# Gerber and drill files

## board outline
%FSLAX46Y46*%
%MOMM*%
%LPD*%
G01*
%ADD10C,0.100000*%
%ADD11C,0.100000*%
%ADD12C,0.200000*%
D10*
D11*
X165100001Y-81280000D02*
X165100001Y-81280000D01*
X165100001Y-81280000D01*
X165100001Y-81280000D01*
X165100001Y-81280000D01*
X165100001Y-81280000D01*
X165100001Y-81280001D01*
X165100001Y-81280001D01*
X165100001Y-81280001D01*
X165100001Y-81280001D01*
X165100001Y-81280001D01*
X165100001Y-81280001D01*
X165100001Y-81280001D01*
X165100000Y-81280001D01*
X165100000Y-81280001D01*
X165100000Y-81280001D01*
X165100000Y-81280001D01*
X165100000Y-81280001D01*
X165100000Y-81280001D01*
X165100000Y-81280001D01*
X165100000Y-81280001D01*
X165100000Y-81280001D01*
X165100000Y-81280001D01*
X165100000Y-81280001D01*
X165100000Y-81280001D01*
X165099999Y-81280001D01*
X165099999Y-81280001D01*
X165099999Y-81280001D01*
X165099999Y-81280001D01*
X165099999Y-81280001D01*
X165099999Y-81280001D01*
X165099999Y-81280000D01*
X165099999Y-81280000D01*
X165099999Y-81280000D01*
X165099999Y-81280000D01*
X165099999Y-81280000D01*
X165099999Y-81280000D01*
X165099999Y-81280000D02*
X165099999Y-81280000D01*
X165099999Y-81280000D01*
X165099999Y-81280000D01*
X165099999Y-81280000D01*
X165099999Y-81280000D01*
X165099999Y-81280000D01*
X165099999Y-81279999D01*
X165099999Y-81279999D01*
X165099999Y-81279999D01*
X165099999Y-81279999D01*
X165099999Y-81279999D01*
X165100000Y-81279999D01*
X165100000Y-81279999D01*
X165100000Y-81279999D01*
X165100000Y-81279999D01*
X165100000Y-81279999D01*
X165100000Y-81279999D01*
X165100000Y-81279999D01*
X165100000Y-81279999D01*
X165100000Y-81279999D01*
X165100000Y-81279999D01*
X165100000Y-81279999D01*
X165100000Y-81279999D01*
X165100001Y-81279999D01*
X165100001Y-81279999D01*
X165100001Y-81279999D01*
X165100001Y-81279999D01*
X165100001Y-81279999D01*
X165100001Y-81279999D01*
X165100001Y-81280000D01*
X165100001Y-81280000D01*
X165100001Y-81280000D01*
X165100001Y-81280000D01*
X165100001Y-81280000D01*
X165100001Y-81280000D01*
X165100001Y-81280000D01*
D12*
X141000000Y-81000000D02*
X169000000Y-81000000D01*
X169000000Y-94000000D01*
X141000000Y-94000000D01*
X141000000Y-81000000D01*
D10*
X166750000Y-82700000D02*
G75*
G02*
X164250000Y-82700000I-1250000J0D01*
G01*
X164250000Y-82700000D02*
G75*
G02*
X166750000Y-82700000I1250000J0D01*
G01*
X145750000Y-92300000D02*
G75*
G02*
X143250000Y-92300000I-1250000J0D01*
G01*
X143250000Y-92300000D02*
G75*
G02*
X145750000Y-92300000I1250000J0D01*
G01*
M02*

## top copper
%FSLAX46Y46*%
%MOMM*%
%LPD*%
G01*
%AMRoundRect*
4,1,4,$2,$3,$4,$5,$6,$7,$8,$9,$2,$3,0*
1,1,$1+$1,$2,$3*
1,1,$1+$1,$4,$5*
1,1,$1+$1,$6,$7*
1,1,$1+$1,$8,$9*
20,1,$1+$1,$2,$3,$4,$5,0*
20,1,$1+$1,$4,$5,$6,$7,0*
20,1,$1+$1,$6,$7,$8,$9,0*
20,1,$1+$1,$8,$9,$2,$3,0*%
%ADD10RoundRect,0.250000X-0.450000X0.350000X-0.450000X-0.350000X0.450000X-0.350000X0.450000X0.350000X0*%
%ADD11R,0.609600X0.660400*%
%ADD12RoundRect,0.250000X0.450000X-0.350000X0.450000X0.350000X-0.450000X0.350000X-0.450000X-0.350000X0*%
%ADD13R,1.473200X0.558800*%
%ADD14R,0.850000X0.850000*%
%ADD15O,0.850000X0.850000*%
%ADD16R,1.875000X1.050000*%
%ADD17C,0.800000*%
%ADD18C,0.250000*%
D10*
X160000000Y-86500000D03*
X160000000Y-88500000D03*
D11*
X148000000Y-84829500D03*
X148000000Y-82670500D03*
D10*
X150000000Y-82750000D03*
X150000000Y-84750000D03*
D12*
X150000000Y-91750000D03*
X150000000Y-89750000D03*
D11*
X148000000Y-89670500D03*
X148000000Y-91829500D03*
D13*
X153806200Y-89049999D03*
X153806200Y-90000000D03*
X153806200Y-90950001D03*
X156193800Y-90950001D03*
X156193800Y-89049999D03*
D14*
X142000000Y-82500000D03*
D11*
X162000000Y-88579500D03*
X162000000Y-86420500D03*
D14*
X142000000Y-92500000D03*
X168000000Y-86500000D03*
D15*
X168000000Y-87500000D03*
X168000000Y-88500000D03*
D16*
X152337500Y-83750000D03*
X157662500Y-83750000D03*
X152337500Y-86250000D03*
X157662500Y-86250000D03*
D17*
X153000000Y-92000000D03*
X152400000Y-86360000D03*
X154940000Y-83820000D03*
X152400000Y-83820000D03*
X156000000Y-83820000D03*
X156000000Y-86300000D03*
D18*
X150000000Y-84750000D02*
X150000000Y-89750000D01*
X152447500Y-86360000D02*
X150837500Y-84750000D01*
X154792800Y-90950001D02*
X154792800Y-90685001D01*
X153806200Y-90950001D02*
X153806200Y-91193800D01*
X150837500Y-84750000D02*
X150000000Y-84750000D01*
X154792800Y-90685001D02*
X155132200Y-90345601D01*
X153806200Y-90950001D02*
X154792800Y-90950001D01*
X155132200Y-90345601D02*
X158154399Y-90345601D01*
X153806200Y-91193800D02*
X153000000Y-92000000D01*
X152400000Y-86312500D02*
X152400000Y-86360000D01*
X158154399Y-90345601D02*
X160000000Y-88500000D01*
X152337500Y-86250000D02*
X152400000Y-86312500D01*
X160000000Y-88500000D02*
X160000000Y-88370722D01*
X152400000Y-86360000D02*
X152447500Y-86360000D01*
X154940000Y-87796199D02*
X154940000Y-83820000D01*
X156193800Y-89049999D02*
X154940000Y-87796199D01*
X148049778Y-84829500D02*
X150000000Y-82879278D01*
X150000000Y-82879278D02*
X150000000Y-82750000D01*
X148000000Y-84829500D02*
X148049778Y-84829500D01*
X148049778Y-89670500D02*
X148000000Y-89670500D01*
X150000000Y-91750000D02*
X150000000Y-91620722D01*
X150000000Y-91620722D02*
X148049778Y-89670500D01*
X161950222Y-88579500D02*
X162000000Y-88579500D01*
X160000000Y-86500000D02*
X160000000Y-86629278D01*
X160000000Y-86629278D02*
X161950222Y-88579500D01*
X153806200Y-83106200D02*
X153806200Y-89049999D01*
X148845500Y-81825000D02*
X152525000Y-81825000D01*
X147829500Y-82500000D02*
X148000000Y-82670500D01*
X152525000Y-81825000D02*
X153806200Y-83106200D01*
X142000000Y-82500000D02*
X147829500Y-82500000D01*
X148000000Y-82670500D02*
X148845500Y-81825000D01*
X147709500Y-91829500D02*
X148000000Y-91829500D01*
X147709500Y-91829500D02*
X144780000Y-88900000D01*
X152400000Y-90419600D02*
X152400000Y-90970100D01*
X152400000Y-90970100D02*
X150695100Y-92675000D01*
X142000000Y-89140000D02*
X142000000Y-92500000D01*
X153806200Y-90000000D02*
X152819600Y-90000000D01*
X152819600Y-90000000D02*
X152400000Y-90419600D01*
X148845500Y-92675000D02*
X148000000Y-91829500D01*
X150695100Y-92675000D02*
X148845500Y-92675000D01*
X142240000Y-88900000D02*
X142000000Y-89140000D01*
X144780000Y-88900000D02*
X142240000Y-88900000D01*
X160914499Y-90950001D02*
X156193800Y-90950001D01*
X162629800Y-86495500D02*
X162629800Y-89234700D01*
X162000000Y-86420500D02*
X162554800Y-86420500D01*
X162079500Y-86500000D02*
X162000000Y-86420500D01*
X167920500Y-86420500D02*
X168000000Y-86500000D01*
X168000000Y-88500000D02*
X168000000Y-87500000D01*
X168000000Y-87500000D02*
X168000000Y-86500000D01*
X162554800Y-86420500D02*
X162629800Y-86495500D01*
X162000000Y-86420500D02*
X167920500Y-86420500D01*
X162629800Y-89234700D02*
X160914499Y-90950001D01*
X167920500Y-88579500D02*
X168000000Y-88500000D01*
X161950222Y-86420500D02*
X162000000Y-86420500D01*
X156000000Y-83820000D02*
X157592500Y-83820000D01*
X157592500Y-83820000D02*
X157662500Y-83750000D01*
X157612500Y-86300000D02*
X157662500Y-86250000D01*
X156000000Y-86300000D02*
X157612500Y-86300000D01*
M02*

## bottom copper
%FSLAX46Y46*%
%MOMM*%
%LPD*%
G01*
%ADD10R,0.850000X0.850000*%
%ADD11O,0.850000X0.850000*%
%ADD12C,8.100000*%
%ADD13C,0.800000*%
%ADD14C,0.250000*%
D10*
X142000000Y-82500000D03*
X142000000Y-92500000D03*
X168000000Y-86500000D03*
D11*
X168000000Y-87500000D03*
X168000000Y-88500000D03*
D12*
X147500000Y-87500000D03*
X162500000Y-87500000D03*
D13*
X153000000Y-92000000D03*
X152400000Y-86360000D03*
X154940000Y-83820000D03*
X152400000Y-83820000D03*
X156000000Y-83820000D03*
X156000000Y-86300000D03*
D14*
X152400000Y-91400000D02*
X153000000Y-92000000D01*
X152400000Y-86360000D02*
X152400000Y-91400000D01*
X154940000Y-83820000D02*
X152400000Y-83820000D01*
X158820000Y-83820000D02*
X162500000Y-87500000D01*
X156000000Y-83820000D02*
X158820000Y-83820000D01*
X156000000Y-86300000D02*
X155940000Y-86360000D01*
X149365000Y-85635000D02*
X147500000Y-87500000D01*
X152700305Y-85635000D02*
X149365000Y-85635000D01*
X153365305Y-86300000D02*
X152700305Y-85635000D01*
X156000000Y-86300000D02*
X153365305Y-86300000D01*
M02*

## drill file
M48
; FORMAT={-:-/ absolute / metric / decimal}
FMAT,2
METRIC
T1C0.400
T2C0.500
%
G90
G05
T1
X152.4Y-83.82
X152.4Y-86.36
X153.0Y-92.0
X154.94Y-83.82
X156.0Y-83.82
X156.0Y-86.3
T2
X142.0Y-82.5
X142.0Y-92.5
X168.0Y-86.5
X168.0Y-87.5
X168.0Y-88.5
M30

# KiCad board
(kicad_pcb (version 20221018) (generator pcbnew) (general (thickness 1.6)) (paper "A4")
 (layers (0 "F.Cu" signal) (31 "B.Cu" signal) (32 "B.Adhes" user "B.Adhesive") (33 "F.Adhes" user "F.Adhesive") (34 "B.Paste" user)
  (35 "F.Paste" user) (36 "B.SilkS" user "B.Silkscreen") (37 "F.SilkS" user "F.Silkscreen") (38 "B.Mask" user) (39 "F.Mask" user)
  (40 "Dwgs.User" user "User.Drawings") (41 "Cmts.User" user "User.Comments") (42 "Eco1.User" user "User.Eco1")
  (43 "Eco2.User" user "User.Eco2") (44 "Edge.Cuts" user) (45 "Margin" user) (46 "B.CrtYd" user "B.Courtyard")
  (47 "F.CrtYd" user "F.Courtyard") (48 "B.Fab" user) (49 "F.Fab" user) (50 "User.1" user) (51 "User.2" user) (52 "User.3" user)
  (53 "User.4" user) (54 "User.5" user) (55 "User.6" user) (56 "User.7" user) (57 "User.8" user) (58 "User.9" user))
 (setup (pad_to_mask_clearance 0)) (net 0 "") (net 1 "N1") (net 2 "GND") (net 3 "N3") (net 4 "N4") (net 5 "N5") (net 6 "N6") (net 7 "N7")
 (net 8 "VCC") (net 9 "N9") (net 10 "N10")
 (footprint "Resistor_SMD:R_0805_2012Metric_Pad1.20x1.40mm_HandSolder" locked (layer "F.Cu") (at 160 87.5 -90)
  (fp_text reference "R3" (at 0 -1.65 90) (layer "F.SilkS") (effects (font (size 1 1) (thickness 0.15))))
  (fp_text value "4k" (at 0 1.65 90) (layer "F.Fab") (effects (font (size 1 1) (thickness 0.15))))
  (pad "1" smd roundrect locked (at -1 0 270) (size 1.2 1.4) (layers "F.Cu" "F.Paste" "F.Mask") (roundrect_rratio 0.208333) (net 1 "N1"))
  (pad "2" smd roundrect locked (at 1 0 270) (size 1.2 1.4) (layers "F.Cu" "F.Paste" "F.Mask") (roundrect_rratio 0.208333) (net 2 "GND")))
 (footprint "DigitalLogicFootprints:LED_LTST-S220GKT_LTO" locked (layer "F.Cu") (at 148 83.75 90)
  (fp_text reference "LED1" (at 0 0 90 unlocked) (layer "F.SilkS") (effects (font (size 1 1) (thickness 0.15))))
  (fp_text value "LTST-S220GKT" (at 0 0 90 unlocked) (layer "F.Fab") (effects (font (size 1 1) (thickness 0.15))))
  (pad "1" smd rect locked (at -1.0795 0 90) (size 0.6604 0.6096) (layers "F.Cu" "F.Paste" "F.Mask") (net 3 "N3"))
  (pad "2" smd rect locked (at 1.0795 0 90) (size 0.6604 0.6096) (layers "F.Cu" "F.Paste" "F.Mask") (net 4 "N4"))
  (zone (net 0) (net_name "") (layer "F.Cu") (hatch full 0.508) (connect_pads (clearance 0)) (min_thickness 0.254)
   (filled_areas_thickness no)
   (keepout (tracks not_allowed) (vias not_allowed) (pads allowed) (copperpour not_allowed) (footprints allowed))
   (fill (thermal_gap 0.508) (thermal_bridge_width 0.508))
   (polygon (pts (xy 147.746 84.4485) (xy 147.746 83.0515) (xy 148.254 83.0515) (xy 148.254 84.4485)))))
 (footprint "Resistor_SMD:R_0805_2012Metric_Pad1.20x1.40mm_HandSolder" (layer "F.Cu") (at 150 83.75 -90)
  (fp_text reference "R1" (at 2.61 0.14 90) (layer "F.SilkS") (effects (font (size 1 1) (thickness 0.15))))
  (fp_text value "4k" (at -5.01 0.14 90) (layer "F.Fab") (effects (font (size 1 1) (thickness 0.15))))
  (pad "1" smd roundrect (at -1 0 270) (size 1.2 1.4) (layers "F.Cu" "F.Paste" "F.Mask") (roundrect_rratio 0.208333) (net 3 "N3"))
  (pad "2" smd roundrect (at 1 0 270) (size 1.2 1.4) (layers "F.Cu" "F.Paste" "F.Mask") (roundrect_rratio 0.208333) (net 2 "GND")))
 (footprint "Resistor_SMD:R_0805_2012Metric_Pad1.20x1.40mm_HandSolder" (layer "F.Cu") (at 150 90.75 90)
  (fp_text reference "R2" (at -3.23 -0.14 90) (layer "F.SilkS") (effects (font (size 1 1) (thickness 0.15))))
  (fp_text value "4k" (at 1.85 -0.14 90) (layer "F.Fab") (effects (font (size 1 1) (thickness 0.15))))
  (pad "1" smd roundrect (at -1 0 90) (size 1.2 1.4) (layers "F.Cu" "F.Paste" "F.Mask") (roundrect_rratio 0.208333) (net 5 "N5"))
  (pad "2" smd roundrect (at 1 0 90) (size 1.2 1.4) (layers "F.Cu" "F.Paste" "F.Mask") (roundrect_rratio 0.208333) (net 2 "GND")))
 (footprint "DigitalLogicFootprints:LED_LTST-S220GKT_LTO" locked (layer "F.Cu") (at 148 90.75 -90)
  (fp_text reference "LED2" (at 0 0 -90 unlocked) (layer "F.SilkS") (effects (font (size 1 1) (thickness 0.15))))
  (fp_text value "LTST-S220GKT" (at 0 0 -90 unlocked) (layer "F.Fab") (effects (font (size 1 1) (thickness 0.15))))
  (pad "1" smd rect locked (at -1.0795 0 270) (size 0.6604 0.6096) (layers "F.Cu" "F.Paste" "F.Mask") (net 5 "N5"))
  (pad "2" smd rect locked (at 1.0795 0 270) (size 0.6604 0.6096) (layers "F.Cu" "F.Paste" "F.Mask") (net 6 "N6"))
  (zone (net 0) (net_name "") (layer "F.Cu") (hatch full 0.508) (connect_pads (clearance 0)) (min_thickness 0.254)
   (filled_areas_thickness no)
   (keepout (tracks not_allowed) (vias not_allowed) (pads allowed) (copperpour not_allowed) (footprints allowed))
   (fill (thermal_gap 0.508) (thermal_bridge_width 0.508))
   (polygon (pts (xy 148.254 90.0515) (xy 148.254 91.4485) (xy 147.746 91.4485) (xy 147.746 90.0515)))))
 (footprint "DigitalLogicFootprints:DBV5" (layer "F.Cu") (at 155 90)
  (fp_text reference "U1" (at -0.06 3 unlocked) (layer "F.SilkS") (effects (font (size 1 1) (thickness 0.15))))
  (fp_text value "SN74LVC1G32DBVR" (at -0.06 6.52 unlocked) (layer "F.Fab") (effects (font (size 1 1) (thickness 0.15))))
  (pad "1" smd rect (at -1.1938 -0.950001) (size 1.4732 0.5588) (layers "F.Cu" "F.Paste" "F.Mask") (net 4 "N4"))
  (pad "2" smd rect (at -1.1938 0) (size 1.4732 0.5588) (layers "F.Cu" "F.Paste" "F.Mask") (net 6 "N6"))
  (pad "3" smd rect (at -1.1938 0.950001) (size 1.4732 0.5588) (layers "F.Cu" "F.Paste" "F.Mask") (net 2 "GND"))
  (pad "4" smd rect (at 1.1938 0.950001) (size 1.4732 0.5588) (layers "F.Cu" "F.Paste" "F.Mask") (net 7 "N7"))
  (pad "5" smd rect (at 1.1938 -0.950001) (size 1.4732 0.5588) (layers "F.Cu" "F.Paste" "F.Mask") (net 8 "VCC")))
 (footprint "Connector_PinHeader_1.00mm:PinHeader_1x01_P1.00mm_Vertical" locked (layer "F.Cu") (at 142 82.5)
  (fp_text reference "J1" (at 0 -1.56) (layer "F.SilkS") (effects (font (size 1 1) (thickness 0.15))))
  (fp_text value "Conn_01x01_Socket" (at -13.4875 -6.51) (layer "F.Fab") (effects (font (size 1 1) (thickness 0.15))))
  (pad "1" thru_hole rect locked (at 0 0) (size 0.85 0.85) (drill 0.5) (layers "*.Cu" "*.Mask") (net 4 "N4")))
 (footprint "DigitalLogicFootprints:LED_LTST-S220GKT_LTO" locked (layer "F.Cu") (at 162 87.5 90)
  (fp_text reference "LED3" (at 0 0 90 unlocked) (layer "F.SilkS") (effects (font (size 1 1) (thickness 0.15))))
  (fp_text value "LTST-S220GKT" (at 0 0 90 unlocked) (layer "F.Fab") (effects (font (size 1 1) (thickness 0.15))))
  (pad "1" smd rect locked (at -1.0795 0 90) (size 0.6604 0.6096) (layers "F.Cu" "F.Paste" "F.Mask") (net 1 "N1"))
  (pad "2" smd rect locked (at 1.0795 0 90) (size 0.6604 0.6096) (layers "F.Cu" "F.Paste" "F.Mask") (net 7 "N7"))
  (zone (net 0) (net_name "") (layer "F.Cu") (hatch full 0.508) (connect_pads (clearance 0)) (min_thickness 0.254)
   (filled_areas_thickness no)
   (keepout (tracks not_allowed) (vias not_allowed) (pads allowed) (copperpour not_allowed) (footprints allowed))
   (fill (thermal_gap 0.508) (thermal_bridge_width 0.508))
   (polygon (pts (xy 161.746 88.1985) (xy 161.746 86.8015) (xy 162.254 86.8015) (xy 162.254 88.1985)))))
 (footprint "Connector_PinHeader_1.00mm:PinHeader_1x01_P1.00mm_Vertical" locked (layer "F.Cu") (at 142 92.5)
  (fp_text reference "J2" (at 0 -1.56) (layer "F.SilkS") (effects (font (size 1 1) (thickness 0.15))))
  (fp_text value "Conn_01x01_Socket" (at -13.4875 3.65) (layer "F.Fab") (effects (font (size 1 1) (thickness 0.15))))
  (pad "1" thru_hole rect locked (at 0 0) (size 0.85 0.85) (drill 0.5) (layers "*.Cu" "*.Mask") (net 6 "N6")))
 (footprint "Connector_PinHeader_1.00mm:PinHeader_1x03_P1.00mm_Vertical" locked (layer "F.Cu") (at 168 86.5)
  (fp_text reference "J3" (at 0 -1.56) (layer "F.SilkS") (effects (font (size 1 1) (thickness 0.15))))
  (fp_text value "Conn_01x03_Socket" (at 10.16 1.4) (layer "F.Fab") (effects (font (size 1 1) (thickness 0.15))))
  (pad "1" thru_hole rect locked (at 0 0) (size 0.85 0.85) (drill 0.5) (layers "*.Cu" "*.Mask") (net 7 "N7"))
  (pad "2" thru_hole oval locked (at 0 1) (size 0.85 0.85) (drill 0.5) (layers "*.Cu" "*.Mask") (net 7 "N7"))
  (pad "3" thru_hole oval locked (at 0 2) (size 0.85 0.85) (drill 0.5) (layers "*.Cu" "*.Mask") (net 7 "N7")))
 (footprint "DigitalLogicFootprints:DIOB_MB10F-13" (layer "F.Cu") (at 155 85)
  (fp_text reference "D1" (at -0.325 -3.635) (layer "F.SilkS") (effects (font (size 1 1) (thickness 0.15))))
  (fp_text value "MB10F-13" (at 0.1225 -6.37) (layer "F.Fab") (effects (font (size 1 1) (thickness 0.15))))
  (pad "1" smd rect (at -2.6625 -1.25) (size 1.875 1.05) (layers "F.Cu" "F.Paste" "F.Mask") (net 8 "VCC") (solder_mask_margin 0.102))
  (pad "2" smd rect (at 2.6625 -1.25 180) (size 1.875 1.05) (layers "F.Cu" "F.Paste" "F.Mask") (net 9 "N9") (solder_mask_margin 0.102))
  (pad "3" smd rect (at -2.6625 1.25) (size 1.875 1.05) (layers "F.Cu" "F.Paste" "F.Mask") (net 2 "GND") (solder_mask_margin 0.102))
  (pad "4" smd rect (at 2.6625 1.25 180) (size 1.875 1.05) (layers "F.Cu" "F.Paste" "F.Mask") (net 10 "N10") (solder_mask_margin 0.102)))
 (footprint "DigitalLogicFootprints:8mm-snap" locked (layer "B.Cu") (at 147.5 87.5 180)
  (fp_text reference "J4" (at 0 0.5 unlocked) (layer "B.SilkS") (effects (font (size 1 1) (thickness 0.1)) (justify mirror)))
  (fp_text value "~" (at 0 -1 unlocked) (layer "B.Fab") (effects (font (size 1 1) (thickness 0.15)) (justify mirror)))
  (pad "1" smd circle locked (at 0 0 180) (size 8.1 8.1) (layers "B.Cu" "B.Paste" "B.Mask") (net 10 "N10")))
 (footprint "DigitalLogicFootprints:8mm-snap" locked (layer "B.Cu") (at 162.5 87.5 180)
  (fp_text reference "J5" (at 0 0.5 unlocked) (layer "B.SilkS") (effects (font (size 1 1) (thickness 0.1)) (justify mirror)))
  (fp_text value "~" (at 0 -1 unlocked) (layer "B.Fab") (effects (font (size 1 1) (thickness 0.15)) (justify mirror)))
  (pad "1" smd circle locked (at 0 0 180) (size 8.1 8.1) (layers "B.Cu" "B.Paste" "B.Mask") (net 9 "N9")))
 (gr_circle (center 165.1 81.28) (end 165.1 81.28) (stroke (width 0.1) (type default)) (fill none) (layer "Edge.Cuts"))
 (gr_rect locked (start 141 81) (end 169 94) (stroke (width 0.2) (type default)) (fill none) (layer "Edge.Cuts"))
 (gr_circle (center 165.5 82.7) (end 166.75 82.7) (stroke (width 0.1) (type default)) (fill none) (layer "Edge.Cuts"))
 (gr_circle (center 144.5 92.3) (end 145.75 92.3) (stroke (width 0.1) (type default)) (fill none) (layer "Edge.Cuts"))
 (segment (start 150 84.75) (end 150 89.75) (width 0.25) (layer "F.Cu") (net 2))
 (segment (start 152.4475 86.36) (end 150.8375 84.75) (width 0.25) (layer "F.Cu") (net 2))
 (segment (start 154.7928 90.950001) (end 154.7928 90.685001) (width 0.25) (layer "F.Cu") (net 2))
 (segment (start 153.8062 90.950001) (end 153.8062 91.1938) (width 0.25) (layer "F.Cu") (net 2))
 (segment (start 150.8375 84.75) (end 150 84.75) (width 0.25) (layer "F.Cu") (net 2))
 (segment (start 154.7928 90.685001) (end 155.1322 90.345601) (width 0.25) (layer "F.Cu") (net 2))
 (segment (start 153.8062 90.950001) (end 154.7928 90.950001) (width 0.25) (layer "F.Cu") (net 2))
 (segment (start 155.1322 90.345601) (end 158.154399 90.345601) (width 0.25) (layer "F.Cu") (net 2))
 (segment (start 153.8062 91.1938) (end 153 92) (width 0.25) (layer "F.Cu") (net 2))
 (segment (start 152.4 86.3125) (end 152.4 86.36) (width 0.25) (layer "F.Cu") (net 2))
 (segment (start 158.154399 90.345601) (end 160 88.5) (width 0.25) (layer "F.Cu") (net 2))
 (segment (start 152.3375 86.25) (end 152.4 86.3125) (width 0.25) (layer "F.Cu") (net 2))
 (segment (start 160 88.5) (end 160 88.370722) (width 0.25) (layer "F.Cu") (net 2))
 (segment (start 152.4 86.36) (end 152.4475 86.36) (width 0.25) (layer "F.Cu") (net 2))
 (via (at 153 92) (size 0.8) (drill 0.4) (layers "F.Cu" "B.Cu") (free) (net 2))
 (via (at 152.4 86.36) (size 0.8) (drill 0.4) (layers "F.Cu" "B.Cu") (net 2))
 (segment (start 152.4 91.4) (end 153 92) (width 0.25) (layer "B.Cu") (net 2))
 (segment (start 152.4 86.36) (end 152.4 91.4) (width 0.25) (layer "B.Cu") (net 2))
 (segment (start 154.94 87.796199) (end 154.94 83.82) (width 0.25) (layer "F.Cu") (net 8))
 (segment (start 156.1938 89.049999) (end 154.94 87.796199) (width 0.25) (layer "F.Cu") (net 8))
 (via (at 154.94 83.82) (size 0.8) (drill 0.4) (layers "F.Cu" "B.Cu") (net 8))
 (via (at 152.4 83.82) (size 0.8) (drill 0.4) (layers "F.Cu" "B.Cu") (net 8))
 (segment (start 154.94 83.82) (end 152.4 83.82) (width 0.25) (layer "B.Cu") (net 8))
 (segment (start 148.049778 84.8295) (end 150 82.879278) (width 0.25) (layer "F.Cu") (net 3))
 (segment (start 150 82.879278) (end 150 82.75) (width 0.25) (layer "F.Cu") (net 3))
 (segment (start 148 84.8295) (end 148.049778 84.8295) (width 0.25) (layer "F.Cu") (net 3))
 (segment (start 148.049778 89.6705) (end 148 89.6705) (width 0.25) (layer "F.Cu") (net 5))
 (segment (start 150 91.75) (end 150 91.620722) (width 0.25) (layer "F.Cu") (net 5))
 (segment (start 150 91.620722) (end 148.049778 89.6705) (width 0.25) (layer "F.Cu") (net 5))
 (segment (start 161.950222 88.5795) (end 162 88.5795) (width 0.25) (layer "F.Cu") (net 1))
 (segment (start 160 86.5) (end 160 86.629278) (width 0.25) (layer "F.Cu") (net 1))
 (segment (start 160 86.629278) (end 161.950222 88.5795) (width 0.25) (layer "F.Cu") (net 1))
 (segment (start 153.8062 83.1062) (end 153.8062 89.049999) (width 0.25) (layer "F.Cu") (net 4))
 (segment (start 148.8455 81.825) (end 152.525 81.825) (width 0.25) (layer "F.Cu") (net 4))
 (segment (start 147.8295 82.5) (end 148 82.6705) (width 0.25) (layer "F.Cu") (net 4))
 (segment (start 152.525 81.825) (end 153.8062 83.1062) (width 0.25) (layer "F.Cu") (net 4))
 (segment (start 142 82.5) (end 147.8295 82.5) (width 0.25) (layer "F.Cu") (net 4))
 (segment (start 148 82.6705) (end 148.8455 81.825) (width 0.25) (layer "F.Cu") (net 4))
 (segment (start 147.7095 91.8295) (end 148 91.8295) (width 0.25) (layer "F.Cu") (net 6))
 (segment (start 147.7095 91.8295) (end 144.78 88.9) (width 0.25) (layer "F.Cu") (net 6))
 (segment (start 152.4 90.4196) (end 152.4 90.9701) (width 0.25) (layer "F.Cu") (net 6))
 (segment (start 152.4 90.9701) (end 150.6951 92.675) (width 0.25) (layer "F.Cu") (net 6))
 (segment (start 142 89.14) (end 142 92.5) (width 0.25) (layer "F.Cu") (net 6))
 (segment (start 153.8062 90) (end 152.8196 90) (width 0.25) (layer "F.Cu") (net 6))
 (segment (start 152.8196 90) (end 152.4 90.4196) (width 0.25) (layer "F.Cu") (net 6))
 (segment (start 148.8455 92.675) (end 148 91.8295) (width 0.25) (layer "F.Cu") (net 6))
 (segment (start 150.6951 92.675) (end 148.8455 92.675) (width 0.25) (layer "F.Cu") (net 6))
 (segment (start 142.24 88.9) (end 142 89.14) (width 0.25) (layer "F.Cu") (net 6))
 (segment (start 144.78 88.9) (end 142.24 88.9) (width 0.25) (layer "F.Cu") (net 6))
 (segment (start 160.914499 90.950001) (end 156.1938 90.950001) (width 0.25) (layer "F.Cu") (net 7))
 (segment (start 162.6298 86.4955) (end 162.6298 89.2347) (width 0.25) (layer "F.Cu") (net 7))
 (segment (start 162 86.4205) (end 162.5548 86.4205) (width 0.25) (layer "F.Cu") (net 7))
 (segment (start 162.0795 86.5) (end 162 86.4205) (width 0.25) (layer "F.Cu") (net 7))
 (segment (start 167.9205 86.4205) (end 168 86.5) (width 0.25) (layer "F.Cu") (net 7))
 (segment (start 168 88.5) (end 168 87.5) (width 0.25) (layer "F.Cu") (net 7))
 (segment (start 168 87.5) (end 168 86.5) (width 0.25) (layer "F.Cu") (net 7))
 (segment (start 162.5548 86.4205) (end 162.6298 86.4955) (width 0.25) (layer "F.Cu") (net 7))
 (segment (start 162 86.4205) (end 167.9205 86.4205) (width 0.25) (layer "F.Cu") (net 7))
 (segment (start 162.6298 89.2347) (end 160.914499 90.950001) (width 0.25) (layer "F.Cu") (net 7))
 (segment (start 167.9205 88.5795) (end 168 88.5) (width 0.25) (layer "F.Cu") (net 7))
 (segment (start 161.950222 86.4205) (end 162 86.4205) (width 0.25) (layer "F.Cu") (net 7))
 (segment (start 156 83.82) (end 157.5925 83.82) (width 0.25) (layer "F.Cu") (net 9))
 (segment (start 157.5925 83.82) (end 157.6625 83.75) (width 0.25) (layer "F.Cu") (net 9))
 (via (at 156 83.82) (size 0.8) (drill 0.4) (layers "F.Cu" "B.Cu") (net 9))
 (segment (start 158.82 83.82) (end 162.5 87.5) (width 0.25) (layer "B.Cu") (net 9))
 (segment (start 156 83.82) (end 158.82 83.82) (width 0.25) (layer "B.Cu") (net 9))
 (segment (start 157.6125 86.3) (end 157.6625 86.25) (width 0.25) (layer "F.Cu") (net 10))
 (segment (start 156 86.3) (end 157.6125 86.3) (width 0.25) (layer "F.Cu") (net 10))
 (via (at 156 86.3) (size 0.8) (drill 0.4) (layers "F.Cu" "B.Cu") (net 10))
 (segment (start 156 86.3) (end 155.94 86.36) (width 0.25) (layer "B.Cu") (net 10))
 (segment (start 149.365 85.635) (end 147.5 87.5) (width 0.25) (layer "B.Cu") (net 10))
 (segment (start 152.700305 85.635) (end 149.365 85.635) (width 0.25) (layer "B.Cu") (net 10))
 (segment (start 153.365305 86.3) (end 152.700305 85.635) (width 0.25) (layer "B.Cu") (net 10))
 (segment (start 156 86.3) (end 153.365305 86.3) (width 0.25) (layer "B.Cu") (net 10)))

